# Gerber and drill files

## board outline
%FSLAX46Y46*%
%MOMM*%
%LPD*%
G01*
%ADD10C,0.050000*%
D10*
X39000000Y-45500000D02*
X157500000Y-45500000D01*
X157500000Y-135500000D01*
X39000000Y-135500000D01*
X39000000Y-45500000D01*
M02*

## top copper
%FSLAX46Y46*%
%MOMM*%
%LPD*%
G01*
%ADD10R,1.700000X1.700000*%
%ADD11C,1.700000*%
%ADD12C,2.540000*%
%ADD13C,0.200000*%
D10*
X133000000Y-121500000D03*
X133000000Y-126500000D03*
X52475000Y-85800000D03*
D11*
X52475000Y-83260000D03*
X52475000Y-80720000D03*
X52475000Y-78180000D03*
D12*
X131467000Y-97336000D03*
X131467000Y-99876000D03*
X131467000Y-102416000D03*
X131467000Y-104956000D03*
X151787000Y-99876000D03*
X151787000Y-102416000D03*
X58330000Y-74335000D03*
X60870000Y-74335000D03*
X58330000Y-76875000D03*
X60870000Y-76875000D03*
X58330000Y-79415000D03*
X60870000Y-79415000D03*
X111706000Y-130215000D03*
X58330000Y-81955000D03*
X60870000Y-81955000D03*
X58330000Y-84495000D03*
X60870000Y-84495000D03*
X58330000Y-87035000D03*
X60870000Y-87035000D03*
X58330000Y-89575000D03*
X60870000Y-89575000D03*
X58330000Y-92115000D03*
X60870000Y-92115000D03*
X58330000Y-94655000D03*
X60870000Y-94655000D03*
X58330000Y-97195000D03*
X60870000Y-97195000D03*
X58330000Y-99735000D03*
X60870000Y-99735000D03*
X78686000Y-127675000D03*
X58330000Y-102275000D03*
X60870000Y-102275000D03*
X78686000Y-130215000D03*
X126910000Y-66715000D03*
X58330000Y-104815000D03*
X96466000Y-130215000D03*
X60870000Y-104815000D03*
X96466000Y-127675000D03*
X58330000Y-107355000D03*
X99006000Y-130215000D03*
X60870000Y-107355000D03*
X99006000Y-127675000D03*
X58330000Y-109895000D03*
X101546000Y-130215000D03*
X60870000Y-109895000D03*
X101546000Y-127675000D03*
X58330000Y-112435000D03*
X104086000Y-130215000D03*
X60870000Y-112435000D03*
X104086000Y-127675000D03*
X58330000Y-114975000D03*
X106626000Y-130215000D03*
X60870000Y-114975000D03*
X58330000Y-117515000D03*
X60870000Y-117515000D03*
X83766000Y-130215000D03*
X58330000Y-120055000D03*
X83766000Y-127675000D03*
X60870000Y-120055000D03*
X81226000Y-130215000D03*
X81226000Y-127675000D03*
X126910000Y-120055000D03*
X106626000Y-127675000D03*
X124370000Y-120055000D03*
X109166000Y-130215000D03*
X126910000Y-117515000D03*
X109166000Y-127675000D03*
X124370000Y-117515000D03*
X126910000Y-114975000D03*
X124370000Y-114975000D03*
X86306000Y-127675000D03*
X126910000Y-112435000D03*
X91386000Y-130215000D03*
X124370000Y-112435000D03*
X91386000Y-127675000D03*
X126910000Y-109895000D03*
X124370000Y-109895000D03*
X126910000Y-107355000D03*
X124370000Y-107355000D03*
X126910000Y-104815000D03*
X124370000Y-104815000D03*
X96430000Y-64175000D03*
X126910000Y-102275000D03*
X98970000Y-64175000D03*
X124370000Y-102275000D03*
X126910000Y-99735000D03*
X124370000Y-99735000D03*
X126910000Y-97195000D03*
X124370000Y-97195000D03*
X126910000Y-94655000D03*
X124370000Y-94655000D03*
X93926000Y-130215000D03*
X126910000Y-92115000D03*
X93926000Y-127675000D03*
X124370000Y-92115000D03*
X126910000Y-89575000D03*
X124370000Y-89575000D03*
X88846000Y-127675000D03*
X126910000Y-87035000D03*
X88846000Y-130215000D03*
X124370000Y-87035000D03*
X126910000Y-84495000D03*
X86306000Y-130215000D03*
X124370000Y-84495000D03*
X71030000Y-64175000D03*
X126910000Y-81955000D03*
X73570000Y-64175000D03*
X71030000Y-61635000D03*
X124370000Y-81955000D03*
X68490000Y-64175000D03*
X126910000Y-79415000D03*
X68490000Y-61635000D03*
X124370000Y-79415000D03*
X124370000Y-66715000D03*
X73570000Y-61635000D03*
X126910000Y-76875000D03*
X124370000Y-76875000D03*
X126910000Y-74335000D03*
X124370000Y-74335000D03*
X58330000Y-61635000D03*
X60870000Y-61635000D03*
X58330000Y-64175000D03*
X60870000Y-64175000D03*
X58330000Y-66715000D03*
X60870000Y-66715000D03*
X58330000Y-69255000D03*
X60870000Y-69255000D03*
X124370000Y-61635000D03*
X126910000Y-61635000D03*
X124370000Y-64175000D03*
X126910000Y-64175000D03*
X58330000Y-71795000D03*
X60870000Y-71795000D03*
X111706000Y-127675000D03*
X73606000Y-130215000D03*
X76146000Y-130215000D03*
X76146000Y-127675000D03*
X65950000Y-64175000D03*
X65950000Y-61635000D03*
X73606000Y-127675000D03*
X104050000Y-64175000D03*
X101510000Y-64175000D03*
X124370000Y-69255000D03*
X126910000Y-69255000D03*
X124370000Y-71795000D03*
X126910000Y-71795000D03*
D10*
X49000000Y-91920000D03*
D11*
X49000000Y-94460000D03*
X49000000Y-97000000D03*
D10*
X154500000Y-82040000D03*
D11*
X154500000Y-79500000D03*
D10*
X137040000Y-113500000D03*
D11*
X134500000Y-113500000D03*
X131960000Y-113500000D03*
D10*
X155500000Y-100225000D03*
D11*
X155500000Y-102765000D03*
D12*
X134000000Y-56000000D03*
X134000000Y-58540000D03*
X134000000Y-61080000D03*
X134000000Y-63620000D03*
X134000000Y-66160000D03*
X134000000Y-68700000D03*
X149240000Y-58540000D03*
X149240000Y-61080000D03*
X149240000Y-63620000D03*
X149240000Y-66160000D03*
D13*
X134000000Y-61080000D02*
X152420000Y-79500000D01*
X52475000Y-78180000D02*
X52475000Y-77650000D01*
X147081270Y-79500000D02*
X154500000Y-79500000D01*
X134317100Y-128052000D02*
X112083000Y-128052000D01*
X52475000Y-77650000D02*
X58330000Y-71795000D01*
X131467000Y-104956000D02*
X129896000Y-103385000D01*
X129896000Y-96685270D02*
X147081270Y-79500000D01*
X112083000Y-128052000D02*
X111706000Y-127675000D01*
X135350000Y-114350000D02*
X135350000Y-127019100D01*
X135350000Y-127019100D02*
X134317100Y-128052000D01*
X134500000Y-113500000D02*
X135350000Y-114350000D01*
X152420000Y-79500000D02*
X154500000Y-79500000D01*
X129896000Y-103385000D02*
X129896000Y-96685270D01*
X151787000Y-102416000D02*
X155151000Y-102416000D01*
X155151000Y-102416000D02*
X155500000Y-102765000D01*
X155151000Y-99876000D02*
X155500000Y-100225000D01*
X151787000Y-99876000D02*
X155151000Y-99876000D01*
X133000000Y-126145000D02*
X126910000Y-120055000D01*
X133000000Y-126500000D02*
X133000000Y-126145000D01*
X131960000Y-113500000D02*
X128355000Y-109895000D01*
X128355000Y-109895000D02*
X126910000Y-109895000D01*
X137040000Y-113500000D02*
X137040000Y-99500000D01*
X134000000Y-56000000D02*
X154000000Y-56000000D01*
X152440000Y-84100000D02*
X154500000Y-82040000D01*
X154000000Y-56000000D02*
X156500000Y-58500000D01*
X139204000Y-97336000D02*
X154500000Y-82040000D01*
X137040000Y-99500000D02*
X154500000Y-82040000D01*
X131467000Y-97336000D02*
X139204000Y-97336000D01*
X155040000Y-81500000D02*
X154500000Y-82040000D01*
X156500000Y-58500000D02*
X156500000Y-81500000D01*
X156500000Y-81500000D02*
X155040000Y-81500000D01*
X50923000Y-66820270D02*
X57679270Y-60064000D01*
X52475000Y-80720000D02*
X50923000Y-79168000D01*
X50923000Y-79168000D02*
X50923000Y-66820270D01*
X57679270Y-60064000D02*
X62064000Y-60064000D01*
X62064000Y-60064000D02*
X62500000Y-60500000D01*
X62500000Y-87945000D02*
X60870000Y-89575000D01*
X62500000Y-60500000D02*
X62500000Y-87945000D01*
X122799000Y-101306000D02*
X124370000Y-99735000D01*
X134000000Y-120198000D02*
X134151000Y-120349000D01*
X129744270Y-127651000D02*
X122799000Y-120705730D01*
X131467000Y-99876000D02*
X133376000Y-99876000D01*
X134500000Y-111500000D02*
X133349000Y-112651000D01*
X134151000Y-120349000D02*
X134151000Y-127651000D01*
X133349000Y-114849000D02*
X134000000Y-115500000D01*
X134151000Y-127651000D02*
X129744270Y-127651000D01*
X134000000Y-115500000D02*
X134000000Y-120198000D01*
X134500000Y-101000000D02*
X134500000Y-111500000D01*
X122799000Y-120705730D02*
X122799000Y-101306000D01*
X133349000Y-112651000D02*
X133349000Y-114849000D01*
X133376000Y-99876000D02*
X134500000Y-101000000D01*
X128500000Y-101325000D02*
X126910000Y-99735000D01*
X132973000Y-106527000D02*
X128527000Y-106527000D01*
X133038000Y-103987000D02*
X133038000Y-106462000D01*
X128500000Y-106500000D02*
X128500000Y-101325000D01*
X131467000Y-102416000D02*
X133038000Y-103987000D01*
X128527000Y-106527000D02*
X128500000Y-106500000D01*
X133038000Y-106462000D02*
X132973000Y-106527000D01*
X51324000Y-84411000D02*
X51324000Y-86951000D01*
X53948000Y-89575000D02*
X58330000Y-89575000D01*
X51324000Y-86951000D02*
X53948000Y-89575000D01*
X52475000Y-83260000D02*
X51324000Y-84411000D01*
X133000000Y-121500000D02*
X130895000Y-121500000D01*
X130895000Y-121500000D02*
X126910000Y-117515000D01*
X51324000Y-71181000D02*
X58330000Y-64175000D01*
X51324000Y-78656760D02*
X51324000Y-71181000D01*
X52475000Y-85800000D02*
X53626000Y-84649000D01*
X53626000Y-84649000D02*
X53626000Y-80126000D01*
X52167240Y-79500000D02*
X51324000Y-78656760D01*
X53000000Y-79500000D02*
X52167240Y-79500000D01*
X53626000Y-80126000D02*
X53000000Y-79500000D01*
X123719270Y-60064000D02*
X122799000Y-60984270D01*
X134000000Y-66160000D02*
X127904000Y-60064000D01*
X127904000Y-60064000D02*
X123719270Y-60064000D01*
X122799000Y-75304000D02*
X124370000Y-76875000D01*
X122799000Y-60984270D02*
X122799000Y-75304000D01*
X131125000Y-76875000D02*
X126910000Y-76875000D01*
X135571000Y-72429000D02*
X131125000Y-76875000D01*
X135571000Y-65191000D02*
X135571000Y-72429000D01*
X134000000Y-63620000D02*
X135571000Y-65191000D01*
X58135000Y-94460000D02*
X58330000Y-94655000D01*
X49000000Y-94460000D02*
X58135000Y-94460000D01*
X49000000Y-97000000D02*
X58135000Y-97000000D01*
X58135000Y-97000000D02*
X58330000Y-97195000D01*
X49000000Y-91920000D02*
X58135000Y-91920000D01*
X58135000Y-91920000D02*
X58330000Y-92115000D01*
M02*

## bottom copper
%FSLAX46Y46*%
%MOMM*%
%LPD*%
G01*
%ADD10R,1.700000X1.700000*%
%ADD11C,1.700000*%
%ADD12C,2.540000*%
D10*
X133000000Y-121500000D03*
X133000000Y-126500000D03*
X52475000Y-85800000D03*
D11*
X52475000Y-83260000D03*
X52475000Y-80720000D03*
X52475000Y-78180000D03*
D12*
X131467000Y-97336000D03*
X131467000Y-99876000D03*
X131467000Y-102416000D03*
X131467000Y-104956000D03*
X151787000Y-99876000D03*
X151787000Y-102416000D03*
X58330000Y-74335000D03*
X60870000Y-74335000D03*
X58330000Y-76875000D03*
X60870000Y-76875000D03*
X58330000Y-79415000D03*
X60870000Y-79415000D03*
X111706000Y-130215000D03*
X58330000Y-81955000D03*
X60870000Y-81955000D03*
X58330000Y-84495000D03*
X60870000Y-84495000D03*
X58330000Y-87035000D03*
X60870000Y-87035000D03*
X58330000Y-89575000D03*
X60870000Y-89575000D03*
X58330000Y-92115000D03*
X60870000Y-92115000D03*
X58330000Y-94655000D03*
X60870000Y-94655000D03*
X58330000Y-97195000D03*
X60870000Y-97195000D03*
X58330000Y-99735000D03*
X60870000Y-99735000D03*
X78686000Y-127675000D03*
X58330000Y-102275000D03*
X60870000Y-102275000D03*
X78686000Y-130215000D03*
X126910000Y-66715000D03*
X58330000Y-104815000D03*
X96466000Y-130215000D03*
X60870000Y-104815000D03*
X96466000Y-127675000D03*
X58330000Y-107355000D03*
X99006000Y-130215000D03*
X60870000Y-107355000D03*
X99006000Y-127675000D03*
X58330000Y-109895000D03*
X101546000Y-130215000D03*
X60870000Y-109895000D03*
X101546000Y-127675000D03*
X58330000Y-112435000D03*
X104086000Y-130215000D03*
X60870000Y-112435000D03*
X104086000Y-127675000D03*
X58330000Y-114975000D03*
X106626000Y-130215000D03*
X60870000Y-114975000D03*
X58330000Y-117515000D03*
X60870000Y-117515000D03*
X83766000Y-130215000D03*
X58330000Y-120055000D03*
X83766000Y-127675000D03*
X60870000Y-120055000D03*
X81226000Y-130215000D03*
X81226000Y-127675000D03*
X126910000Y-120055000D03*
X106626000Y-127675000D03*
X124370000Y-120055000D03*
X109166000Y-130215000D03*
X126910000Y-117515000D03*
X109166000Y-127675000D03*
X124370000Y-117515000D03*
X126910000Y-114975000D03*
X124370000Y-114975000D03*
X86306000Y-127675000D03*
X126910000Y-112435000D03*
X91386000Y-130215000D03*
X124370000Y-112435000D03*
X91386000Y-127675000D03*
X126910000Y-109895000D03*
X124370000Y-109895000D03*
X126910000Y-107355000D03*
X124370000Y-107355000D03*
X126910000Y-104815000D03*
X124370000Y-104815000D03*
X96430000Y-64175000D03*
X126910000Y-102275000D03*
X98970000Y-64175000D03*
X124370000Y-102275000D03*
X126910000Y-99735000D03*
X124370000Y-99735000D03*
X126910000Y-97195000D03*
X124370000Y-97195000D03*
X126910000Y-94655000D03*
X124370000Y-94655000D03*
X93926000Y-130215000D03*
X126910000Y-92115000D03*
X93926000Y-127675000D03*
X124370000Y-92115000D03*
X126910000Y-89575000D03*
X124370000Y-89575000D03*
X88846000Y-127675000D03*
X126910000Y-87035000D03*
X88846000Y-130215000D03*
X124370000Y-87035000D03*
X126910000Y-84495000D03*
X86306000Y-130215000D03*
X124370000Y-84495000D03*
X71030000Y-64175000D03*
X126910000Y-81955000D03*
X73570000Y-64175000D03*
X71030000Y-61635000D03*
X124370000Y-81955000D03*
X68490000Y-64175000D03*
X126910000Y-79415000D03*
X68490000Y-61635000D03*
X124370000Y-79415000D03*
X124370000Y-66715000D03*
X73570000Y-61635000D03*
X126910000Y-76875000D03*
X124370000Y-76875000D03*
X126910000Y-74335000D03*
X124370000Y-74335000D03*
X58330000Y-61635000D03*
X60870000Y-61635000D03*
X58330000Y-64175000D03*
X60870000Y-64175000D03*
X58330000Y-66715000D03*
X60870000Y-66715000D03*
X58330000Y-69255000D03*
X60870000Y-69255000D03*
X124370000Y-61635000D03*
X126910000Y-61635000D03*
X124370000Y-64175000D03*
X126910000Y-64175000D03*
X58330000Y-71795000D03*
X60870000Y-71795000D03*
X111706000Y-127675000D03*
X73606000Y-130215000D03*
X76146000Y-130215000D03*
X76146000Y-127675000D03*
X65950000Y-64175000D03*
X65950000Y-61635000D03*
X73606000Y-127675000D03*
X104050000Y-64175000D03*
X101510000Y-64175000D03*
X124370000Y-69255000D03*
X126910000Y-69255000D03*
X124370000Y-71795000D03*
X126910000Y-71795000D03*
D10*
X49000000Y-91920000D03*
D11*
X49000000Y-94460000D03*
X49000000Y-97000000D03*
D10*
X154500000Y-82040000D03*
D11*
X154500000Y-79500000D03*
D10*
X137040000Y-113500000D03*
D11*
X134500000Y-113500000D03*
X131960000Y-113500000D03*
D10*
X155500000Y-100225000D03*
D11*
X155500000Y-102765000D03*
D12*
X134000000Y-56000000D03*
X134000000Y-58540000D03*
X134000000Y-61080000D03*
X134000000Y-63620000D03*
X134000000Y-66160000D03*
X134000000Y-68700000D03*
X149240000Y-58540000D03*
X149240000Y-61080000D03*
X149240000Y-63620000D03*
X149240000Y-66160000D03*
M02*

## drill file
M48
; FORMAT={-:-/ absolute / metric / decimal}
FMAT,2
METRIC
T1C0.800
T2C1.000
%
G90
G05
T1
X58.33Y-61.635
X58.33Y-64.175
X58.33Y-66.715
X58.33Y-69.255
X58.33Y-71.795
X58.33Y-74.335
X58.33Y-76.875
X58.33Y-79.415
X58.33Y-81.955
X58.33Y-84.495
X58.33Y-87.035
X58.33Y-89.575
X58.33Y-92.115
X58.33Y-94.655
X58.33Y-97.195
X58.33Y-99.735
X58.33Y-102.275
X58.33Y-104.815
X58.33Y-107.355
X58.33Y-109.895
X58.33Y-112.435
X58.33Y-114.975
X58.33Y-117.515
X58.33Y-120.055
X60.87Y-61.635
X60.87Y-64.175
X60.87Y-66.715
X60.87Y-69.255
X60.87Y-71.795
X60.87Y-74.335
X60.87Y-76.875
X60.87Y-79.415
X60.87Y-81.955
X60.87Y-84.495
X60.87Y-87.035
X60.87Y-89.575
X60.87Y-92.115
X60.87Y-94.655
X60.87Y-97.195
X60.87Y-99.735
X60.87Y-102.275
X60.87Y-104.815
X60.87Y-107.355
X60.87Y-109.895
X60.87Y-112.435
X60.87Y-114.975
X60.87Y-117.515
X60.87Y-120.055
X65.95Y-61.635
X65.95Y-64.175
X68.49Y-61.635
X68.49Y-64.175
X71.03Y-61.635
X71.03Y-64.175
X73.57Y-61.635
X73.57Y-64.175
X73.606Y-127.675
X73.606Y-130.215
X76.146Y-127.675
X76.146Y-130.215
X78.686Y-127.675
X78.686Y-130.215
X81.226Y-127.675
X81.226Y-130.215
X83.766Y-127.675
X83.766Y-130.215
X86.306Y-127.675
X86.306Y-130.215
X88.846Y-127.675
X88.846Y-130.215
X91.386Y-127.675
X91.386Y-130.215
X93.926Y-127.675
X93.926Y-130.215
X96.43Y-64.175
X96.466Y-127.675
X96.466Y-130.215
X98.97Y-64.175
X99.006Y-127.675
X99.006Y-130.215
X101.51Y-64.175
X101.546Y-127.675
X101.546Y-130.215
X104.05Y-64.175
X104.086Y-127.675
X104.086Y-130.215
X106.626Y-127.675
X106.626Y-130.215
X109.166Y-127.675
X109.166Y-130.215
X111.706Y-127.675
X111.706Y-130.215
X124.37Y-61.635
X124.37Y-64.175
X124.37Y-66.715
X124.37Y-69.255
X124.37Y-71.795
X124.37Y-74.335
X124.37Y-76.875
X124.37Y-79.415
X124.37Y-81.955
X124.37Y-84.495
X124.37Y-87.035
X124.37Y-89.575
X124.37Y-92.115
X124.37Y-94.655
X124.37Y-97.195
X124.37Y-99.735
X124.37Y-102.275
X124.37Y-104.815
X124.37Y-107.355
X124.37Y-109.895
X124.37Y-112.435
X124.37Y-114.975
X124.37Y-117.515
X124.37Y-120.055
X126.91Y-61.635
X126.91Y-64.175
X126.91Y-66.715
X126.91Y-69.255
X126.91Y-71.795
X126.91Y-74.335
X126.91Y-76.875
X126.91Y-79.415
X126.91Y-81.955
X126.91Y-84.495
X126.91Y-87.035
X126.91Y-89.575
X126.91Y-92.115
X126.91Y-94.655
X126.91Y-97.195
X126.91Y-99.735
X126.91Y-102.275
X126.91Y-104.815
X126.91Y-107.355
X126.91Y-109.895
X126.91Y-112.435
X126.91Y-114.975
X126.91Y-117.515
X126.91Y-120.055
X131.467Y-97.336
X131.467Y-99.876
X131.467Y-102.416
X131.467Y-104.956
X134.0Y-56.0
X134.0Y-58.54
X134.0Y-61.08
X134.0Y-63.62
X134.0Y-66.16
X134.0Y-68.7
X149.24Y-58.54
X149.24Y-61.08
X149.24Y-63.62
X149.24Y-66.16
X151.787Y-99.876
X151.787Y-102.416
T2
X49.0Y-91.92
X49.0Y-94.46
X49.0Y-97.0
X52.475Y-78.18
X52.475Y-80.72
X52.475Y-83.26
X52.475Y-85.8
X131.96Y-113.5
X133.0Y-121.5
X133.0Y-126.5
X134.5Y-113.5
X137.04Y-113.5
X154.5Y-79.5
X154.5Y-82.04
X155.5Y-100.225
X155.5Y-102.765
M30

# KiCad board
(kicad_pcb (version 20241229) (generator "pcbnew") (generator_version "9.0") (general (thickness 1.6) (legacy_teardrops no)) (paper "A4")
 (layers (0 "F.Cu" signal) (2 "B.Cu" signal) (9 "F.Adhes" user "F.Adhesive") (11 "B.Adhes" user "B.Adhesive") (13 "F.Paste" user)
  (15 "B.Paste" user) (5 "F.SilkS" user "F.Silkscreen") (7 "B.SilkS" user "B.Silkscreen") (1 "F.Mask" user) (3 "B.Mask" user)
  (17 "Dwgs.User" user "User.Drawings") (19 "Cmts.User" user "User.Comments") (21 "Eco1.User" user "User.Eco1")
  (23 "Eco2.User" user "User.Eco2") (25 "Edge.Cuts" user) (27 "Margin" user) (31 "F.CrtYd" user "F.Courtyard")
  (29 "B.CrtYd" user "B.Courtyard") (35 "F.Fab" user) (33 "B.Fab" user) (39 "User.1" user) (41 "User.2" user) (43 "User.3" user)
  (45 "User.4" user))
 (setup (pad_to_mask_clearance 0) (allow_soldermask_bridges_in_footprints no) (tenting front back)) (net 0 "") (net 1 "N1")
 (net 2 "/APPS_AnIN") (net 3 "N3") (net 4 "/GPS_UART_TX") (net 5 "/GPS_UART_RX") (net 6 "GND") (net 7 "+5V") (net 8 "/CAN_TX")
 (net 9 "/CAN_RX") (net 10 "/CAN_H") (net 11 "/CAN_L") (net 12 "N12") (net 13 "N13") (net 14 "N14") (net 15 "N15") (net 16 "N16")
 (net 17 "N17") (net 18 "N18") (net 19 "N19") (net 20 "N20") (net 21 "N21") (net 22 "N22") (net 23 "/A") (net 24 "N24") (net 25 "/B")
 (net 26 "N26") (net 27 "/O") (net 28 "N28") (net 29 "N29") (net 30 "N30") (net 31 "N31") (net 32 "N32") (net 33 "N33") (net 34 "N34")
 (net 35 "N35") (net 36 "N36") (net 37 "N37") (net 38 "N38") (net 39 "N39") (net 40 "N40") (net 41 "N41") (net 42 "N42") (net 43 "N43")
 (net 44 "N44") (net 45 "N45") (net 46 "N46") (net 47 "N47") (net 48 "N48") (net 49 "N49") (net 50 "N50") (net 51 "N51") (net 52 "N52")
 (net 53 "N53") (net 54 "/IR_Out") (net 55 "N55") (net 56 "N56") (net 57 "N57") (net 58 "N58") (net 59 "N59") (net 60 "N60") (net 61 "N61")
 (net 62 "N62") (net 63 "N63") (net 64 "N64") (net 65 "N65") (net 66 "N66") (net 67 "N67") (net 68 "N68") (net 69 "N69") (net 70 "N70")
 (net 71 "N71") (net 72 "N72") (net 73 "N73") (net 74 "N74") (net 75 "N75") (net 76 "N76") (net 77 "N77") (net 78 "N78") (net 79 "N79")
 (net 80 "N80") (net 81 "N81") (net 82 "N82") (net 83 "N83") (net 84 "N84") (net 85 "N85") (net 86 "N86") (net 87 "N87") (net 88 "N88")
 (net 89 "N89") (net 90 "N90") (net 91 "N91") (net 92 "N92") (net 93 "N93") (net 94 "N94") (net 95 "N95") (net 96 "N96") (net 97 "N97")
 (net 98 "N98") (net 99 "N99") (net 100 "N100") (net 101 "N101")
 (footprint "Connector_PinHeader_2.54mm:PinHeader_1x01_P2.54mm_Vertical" (layer "F.Cu") (at 133 121.5)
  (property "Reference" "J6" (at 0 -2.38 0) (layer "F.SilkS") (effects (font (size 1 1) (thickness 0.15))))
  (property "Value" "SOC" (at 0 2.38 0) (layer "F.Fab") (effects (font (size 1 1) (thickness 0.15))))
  (pad "1" thru_hole rect (at 0 0) (size 1.7 1.7) (drill 1) (layers "*.Cu" "*.Mask") (remove_unused_layers no) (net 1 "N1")))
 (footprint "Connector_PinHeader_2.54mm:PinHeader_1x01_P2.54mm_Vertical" (layer "F.Cu") (at 133 126.5)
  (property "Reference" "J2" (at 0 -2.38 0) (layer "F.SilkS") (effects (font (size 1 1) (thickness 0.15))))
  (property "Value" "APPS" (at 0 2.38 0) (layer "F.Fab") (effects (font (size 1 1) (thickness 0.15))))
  (pad "1" thru_hole rect (at 0 0) (size 1.7 1.7) (drill 1) (layers "*.Cu" "*.Mask") (remove_unused_layers no) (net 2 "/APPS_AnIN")))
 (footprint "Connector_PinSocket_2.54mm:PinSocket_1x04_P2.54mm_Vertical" (layer "F.Cu") (at 52.475 85.8 180)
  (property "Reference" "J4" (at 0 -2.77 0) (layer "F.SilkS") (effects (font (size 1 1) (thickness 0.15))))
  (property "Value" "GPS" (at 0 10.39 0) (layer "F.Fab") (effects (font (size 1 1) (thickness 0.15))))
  (pad "1" thru_hole rect (at 0 0 180) (size 1.7 1.7) (drill 1) (layers "*.Cu" "*.Mask") (remove_unused_layers no) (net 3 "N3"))
  (pad "2" thru_hole circle (at 0 2.54 180) (size 1.7 1.7) (drill 1) (layers "*.Cu" "*.Mask") (remove_unused_layers no)
   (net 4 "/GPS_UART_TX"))
  (pad "3" thru_hole circle (at 0 5.08 180) (size 1.7 1.7) (drill 1) (layers "*.Cu" "*.Mask") (remove_unused_layers no)
   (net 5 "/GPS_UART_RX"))
  (pad "4" thru_hole circle (at 0 7.62 180) (size 1.7 1.7) (drill 1) (layers "*.Cu" "*.Mask") (remove_unused_layers no) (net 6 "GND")))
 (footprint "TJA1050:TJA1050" (layer "F.Cu") (at 141.627 107.242)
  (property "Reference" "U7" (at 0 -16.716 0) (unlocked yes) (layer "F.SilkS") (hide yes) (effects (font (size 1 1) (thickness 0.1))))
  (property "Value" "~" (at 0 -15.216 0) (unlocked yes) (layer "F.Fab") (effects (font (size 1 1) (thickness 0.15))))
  (pad "1" thru_hole circle (at -10.16 -9.906) (size 2.54 2.54) (drill 0.8) (layers "*.Cu" "*.Mask") (remove_unused_layers no) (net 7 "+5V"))
  (pad "2" thru_hole circle (at -10.16 -7.366) (size 2.54 2.54) (drill 0.8) (layers "*.Cu" "*.Mask") (remove_unused_layers no)
   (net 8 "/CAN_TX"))
  (pad "3" thru_hole circle (at -10.16 -4.826) (size 2.54 2.54) (drill 0.8) (layers "*.Cu" "*.Mask") (remove_unused_layers no)
   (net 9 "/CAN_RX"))
  (pad "4" thru_hole circle (at -10.16 -2.286) (size 2.54 2.54) (drill 0.8) (layers "*.Cu" "*.Mask") (remove_unused_layers no) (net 6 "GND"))
  (pad "5" thru_hole circle (at 10.16 -7.366) (size 2.54 2.54) (drill 0.8) (layers "*.Cu" "*.Mask") (remove_unused_layers no)
   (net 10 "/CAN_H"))
  (pad "6" thru_hole circle (at 10.16 -4.826) (size 2.54 2.54) (drill 0.8) (layers "*.Cu" "*.Mask") (remove_unused_layers no)
   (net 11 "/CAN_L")))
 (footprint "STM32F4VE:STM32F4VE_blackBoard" (layer "F.Cu") (at 92.62 89.575)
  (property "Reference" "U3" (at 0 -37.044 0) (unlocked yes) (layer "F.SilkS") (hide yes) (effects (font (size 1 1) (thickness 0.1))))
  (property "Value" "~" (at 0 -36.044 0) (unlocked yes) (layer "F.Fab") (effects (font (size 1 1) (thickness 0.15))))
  (pad "1" thru_hole circle (at -34.29 -15.24) (size 2.54 2.54) (drill 0.8) (layers "*.Cu" "*.Mask") (remove_unused_layers no)
   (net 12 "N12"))
  (pad "2" thru_hole circle (at -31.75 -15.24) (size 2.54 2.54) (drill 0.8) (layers "*.Cu" "*.Mask") (remove_unused_layers no)
   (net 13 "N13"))
  (pad "3" thru_hole circle (at -34.29 -12.7) (size 2.54 2.54) (drill 0.8) (layers "*.Cu" "*.Mask") (remove_unused_layers no) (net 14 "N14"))
  (pad "4" thru_hole circle (at -31.75 -12.7) (size 2.54 2.54) (drill 0.8) (layers "*.Cu" "*.Mask") (remove_unused_layers no) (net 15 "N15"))
  (pad "5" thru_hole circle (at -34.29 -10.16) (size 2.54 2.54) (drill 0.8) (layers "*.Cu" "*.Mask") (remove_unused_layers no)
   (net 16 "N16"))
  (pad "7" thru_hole circle (at -31.75 -10.16) (size 2.54 2.54) (drill 0.8) (layers "*.Cu" "*.Mask") (remove_unused_layers no)
   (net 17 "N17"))
  (pad "14" thru_hole circle (at 19.086 40.64) (size 2.54 2.54) (drill 0.8) (layers "*.Cu" "*.Mask") (remove_unused_layers no)
   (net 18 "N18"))
  (pad "15" thru_hole circle (at -34.29 -7.62) (size 2.54 2.54) (drill 0.8) (layers "*.Cu" "*.Mask") (remove_unused_layers no)
   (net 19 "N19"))
  (pad "16" thru_hole circle (at -31.75 -7.62) (size 2.54 2.54) (drill 0.8) (layers "*.Cu" "*.Mask") (remove_unused_layers no)
   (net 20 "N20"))
  (pad "17" thru_hole circle (at -34.29 -5.08) (size 2.54 2.54) (drill 0.8) (layers "*.Cu" "*.Mask") (remove_unused_layers no)
   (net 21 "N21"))
  (pad "18" thru_hole circle (at -31.75 -5.08) (size 2.54 2.54) (drill 0.8) (layers "*.Cu" "*.Mask") (remove_unused_layers no)
   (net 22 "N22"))
  (pad "20" thru_hole circle (at -34.29 -2.54) (size 2.54 2.54) (drill 0.8) (layers "*.Cu" "*.Mask") (remove_unused_layers no))
  (pad "21" thru_hole circle (at -31.75 -2.54) (size 2.54 2.54) (drill 0.8) (layers "*.Cu" "*.Mask") (remove_unused_layers no))
  (pad "23" thru_hole circle (at -34.29 0) (size 2.54 2.54) (drill 0.8) (layers "*.Cu" "*.Mask") (remove_unused_layers no)
   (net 4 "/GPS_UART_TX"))
  (pad "24" thru_hole circle (at -31.75 0) (size 2.54 2.54) (drill 0.8) (layers "*.Cu" "*.Mask") (remove_unused_layers no)
   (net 5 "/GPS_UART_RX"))
  (pad "25" thru_hole circle (at -34.29 2.54) (size 2.54 2.54) (drill 0.8) (layers "*.Cu" "*.Mask") (remove_unused_layers no) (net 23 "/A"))
  (pad "26" thru_hole circle (at -31.75 2.54) (size 2.54 2.54) (drill 0.8) (layers "*.Cu" "*.Mask") (remove_unused_layers no) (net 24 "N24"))
  (pad "29" thru_hole circle (at -34.29 5.08) (size 2.54 2.54) (drill 0.8) (layers "*.Cu" "*.Mask") (remove_unused_layers no) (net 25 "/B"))
  (pad "30" thru_hole circle (at -31.75 5.08) (size 2.54 2.54) (drill 0.8) (layers "*.Cu" "*.Mask") (remove_unused_layers no) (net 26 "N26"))
  (pad "31" thru_hole circle (at -34.29 7.62) (size 2.54 2.54) (drill 0.8) (layers "*.Cu" "*.Mask") (remove_unused_layers no) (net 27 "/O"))
  (pad "32" thru_hole circle (at -31.75 7.62) (size 2.54 2.54) (drill 0.8) (layers "*.Cu" "*.Mask") (remove_unused_layers no) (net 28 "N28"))
  (pad "33" thru_hole circle (at -34.29 10.16) (size 2.54 2.54) (drill 0.8) (layers "*.Cu" "*.Mask") (remove_unused_layers no)
   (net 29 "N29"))
  (pad "34" thru_hole circle (at -31.75 10.16) (size 2.54 2.54) (drill 0.8) (layers "*.Cu" "*.Mask") (remove_unused_layers no)
   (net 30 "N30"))
  (pad "34" thru_hole circle (at -13.934 38.1) (size 2.54 2.54) (drill 0.8) (layers "*.Cu" "*.Mask") (remove_unused_layers no)
   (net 30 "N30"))
  (pad "35" thru_hole circle (at -34.29 12.7) (size 2.54 2.54) (drill 0.8) (layers "*.Cu" "*.Mask") (remove_unused_layers no) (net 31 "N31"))
  (pad "36" thru_hole circle (at -31.75 12.7) (size 2.54 2.54) (drill 0.8) (layers "*.Cu" "*.Mask") (remove_unused_layers no) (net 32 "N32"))
  (pad "36" thru_hole circle (at -13.934 40.64) (size 2.54 2.54) (drill 0.8) (layers "*.Cu" "*.Mask") (remove_unused_layers no)
   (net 32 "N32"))
  (pad "37" thru_hole circle (at 34.29 -22.86) (size 2.54 2.54) (drill 0.8) (layers "*.Cu" "*.Mask") (remove_unused_layers no)
   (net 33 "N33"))
  (pad "38" thru_hole circle (at -34.29 15.24) (size 2.54 2.54) (drill 0.8) (layers "*.Cu" "*.Mask") (remove_unused_layers no)
   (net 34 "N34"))
  (pad "38" thru_hole circle (at 3.846 40.64) (size 2.54 2.54) (drill 0.8) (layers "*.Cu" "*.Mask") (remove_unused_layers no) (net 34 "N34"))
  (pad "39" thru_hole circle (at -31.75 15.24) (size 2.54 2.54) (drill 0.8) (layers "*.Cu" "*.Mask") (remove_unused_layers no)
   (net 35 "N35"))
  (pad "39" thru_hole circle (at 3.846 38.1) (size 2.54 2.54) (drill 0.8) (layers "*.Cu" "*.Mask") (remove_unused_layers no) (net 35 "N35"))
  (pad "40" thru_hole circle (at -34.29 17.78) (size 2.54 2.54) (drill 0.8) (layers "*.Cu" "*.Mask") (remove_unused_layers no)
   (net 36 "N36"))
  (pad "40" thru_hole circle (at 6.386 40.64) (size 2.54 2.54) (drill 0.8) (layers "*.Cu" "*.Mask") (remove_unused_layers no) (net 36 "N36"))
  (pad "41" thru_hole circle (at -31.75 17.78) (size 2.54 2.54) (drill 0.8) (layers "*.Cu" "*.Mask") (remove_unused_layers no)
   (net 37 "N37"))
  (pad "41" thru_hole circle (at 6.386 38.1) (size 2.54 2.54) (drill 0.8) (layers "*.Cu" "*.Mask") (remove_unused_layers no) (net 37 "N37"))
  (pad "42" thru_hole circle (at -34.29 20.32) (size 2.54 2.54) (drill 0.8) (layers "*.Cu" "*.Mask") (remove_unused_layers no)
   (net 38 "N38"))
  (pad "42" thru_hole circle (at 8.926 40.64) (size 2.54 2.54) (drill 0.8) (layers "*.Cu" "*.Mask") (remove_unused_layers no) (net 38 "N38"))
  (pad "43" thru_hole circle (at -31.75 20.32) (size 2.54 2.54) (drill 0.8) (layers "*.Cu" "*.Mask") (remove_unused_layers no)
   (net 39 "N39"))
  (pad "43" thru_hole circle (at 8.926 38.1) (size 2.54 2.54) (drill 0.8) (layers "*.Cu" "*.Mask") (remove_unused_layers no) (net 39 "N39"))
  (pad "44" thru_hole circle (at -34.29 22.86) (size 2.54 2.54) (drill 0.8) (layers "*.Cu" "*.Mask") (remove_unused_layers no)
   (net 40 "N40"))
  (pad "44" thru_hole circle (at 11.466 40.64) (size 2.54 2.54) (drill 0.8) (layers "*.Cu" "*.Mask") (remove_unused_layers no)
   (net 40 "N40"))
  (pad "45" thru_hole circle (at -31.75 22.86) (size 2.54 2.54) (drill 0.8) (layers "*.Cu" "*.Mask") (remove_unused_layers no)
   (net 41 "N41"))
  (pad "45" thru_hole circle (at 11.466 38.1) (size 2.54 2.54) (drill 0.8) (layers "*.Cu" "*.Mask") (remove_unused_layers no) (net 41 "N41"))
  (pad "46" thru_hole circle (at -34.29 25.4) (size 2.54 2.54) (drill 0.8) (layers "*.Cu" "*.Mask") (remove_unused_layers no) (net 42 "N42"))
  (pad "46" thru_hole circle (at 14.006 40.64) (size 2.54 2.54) (drill 0.8) (layers "*.Cu" "*.Mask") (remove_unused_layers no)
   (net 42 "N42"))
  (pad "47" thru_hole circle (at -31.75 25.4) (size 2.54 2.54) (drill 0.8) (layers "*.Cu" "*.Mask") (remove_unused_layers no) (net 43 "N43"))
  (pad "48" thru_hole circle (at -34.29 27.94) (size 2.54 2.54) (drill 0.8) (layers "*.Cu" "*.Mask") (remove_unused_layers no)
   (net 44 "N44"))
  (pad "51" thru_hole circle (at -31.75 27.94) (size 2.54 2.54) (drill 0.8) (layers "*.Cu" "*.Mask") (remove_unused_layers no)
   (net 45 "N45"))
  (pad "51" thru_hole circle (at -8.854 40.64) (size 2.54 2.54) (drill 0.8) (layers "*.Cu" "*.Mask") (remove_unused_layers no)
   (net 45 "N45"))
  (pad "52" thru_hole circle (at -34.29 30.48) (size 2.54 2.54) (drill 0.8) (layers "*.Cu" "*.Mask") (remove_unused_layers no)
   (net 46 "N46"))
  (pad "52" thru_hole circle (at -8.854 38.1) (size 2.54 2.54) (drill 0.8) (layers "*.Cu" "*.Mask") (remove_unused_layers no) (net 46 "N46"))
  (pad "53" thru_hole circle (at -31.75 30.48) (size 2.54 2.54) (drill 0.8) (layers "*.Cu" "*.Mask") (remove_unused_layers no)
   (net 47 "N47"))
  (pad "53" thru_hole circle (at -11.394 40.64) (size 2.54 2.54) (drill 0.8) (layers "*.Cu" "*.Mask") (remove_unused_layers no)
   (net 47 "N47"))
  (pad "54" thru_hole circle (at -11.394 38.1) (size 2.54 2.54) (drill 0.8) (layers "*.Cu" "*.Mask") (remove_unused_layers no)
   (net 2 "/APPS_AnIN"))
  (pad "54" thru_hole circle (at 34.29 30.48) (size 2.54 2.54) (drill 0.8) (layers "*.Cu" "*.Mask") (remove_unused_layers no)
   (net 2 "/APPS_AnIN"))
  (pad "55" thru_hole circle (at 14.006 38.1) (size 2.54 2.54) (drill 0.8) (layers "*.Cu" "*.Mask") (remove_unused_layers no) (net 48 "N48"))
  (pad "55" thru_hole circle (at 31.75 30.48) (size 2.54 2.54) (drill 0.8) (layers "*.Cu" "*.Mask") (remove_unused_layers no) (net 48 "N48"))
  (pad "56" thru_hole circle (at 16.546 40.64) (size 2.54 2.54) (drill 0.8) (layers "*.Cu" "*.Mask") (remove_unused_layers no) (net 1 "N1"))
  (pad "56" thru_hole circle (at 34.29 27.94) (size 2.54 2.54) (drill 0.8) (layers "*.Cu" "*.Mask") (remove_unused_layers no) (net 1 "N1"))
  (pad "57" thru_hole circle (at 16.546 38.1) (size 2.54 2.54) (drill 0.8) (layers "*.Cu" "*.Mask") (remove_unused_layers no) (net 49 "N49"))
  (pad "57" thru_hole circle (at 31.75 27.94) (size 2.54 2.54) (drill 0.8) (layers "*.Cu" "*.Mask") (remove_unused_layers no) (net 49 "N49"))
  (pad "58" thru_hole circle (at 34.29 25.4) (size 2.54 2.54) (drill 0.8) (layers "*.Cu" "*.Mask") (remove_unused_layers no) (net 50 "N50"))
  (pad "59" thru_hole circle (at 31.75 25.4) (size 2.54 2.54) (drill 0.8) (layers "*.Cu" "*.Mask") (remove_unused_layers no) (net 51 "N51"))
  (pad "60" thru_hole circle (at -6.314 38.1) (size 2.54 2.54) (drill 0.8) (layers "*.Cu" "*.Mask") (remove_unused_layers no) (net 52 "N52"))
  (pad "60" thru_hole circle (at 34.29 22.86) (size 2.54 2.54) (drill 0.8) (layers "*.Cu" "*.Mask") (remove_unused_layers no) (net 52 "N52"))
  (pad "61" thru_hole circle (at -1.234 40.64) (size 2.54 2.54) (drill 0.8) (layers "*.Cu" "*.Mask") (remove_unused_layers no)
   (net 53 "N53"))
  (pad "61" thru_hole circle (at 31.75 22.86) (size 2.54 2.54) (drill 0.8) (layers "*.Cu" "*.Mask") (remove_unused_layers no) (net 53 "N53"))
  (pad "62" thru_hole circle (at -1.234 38.1) (size 2.54 2.54) (drill 0.8) (layers "*.Cu" "*.Mask") (remove_unused_layers no)
   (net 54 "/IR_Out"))
  (pad "62" thru_hole circle (at 34.29 20.32) (size 2.54 2.54) (drill 0.8) (layers "*.Cu" "*.Mask") (remove_unused_layers no)
   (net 54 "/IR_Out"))
  (pad "63" thru_hole circle (at 31.75 20.32) (size 2.54 2.54) (drill 0.8) (layers "*.Cu" "*.Mask") (remove_unused_layers no) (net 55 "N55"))
  (pad "64" thru_hole circle (at 34.29 17.78) (size 2.54 2.54) (drill 0.8) (layers "*.Cu" "*.Mask") (remove_unused_layers no) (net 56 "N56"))
  (pad "65" thru_hole circle (at 31.75 17.78) (size 2.54 2.54) (drill 0.8) (layers "*.Cu" "*.Mask") (remove_unused_layers no) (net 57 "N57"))
  (pad "66" thru_hole circle (at 34.29 15.24) (size 2.54 2.54) (drill 0.8) (layers "*.Cu" "*.Mask") (remove_unused_layers no) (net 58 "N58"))
  (pad "67" thru_hole circle (at 31.75 15.24) (size 2.54 2.54) (drill 0.8) (layers "*.Cu" "*.Mask") (remove_unused_layers no) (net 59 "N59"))
  (pad "68" thru_hole circle (at 3.81 -25.4) (size 2.54 2.54) (drill 0.8) (layers "*.Cu" "*.Mask") (remove_unused_layers no) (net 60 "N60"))
  (pad "68" thru_hole circle (at 34.29 12.7) (size 2.54 2.54) (drill 0.8) (layers "*.Cu" "*.Mask") (remove_unused_layers no) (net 60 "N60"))
  (pad "69" thru_hole circle (at 6.35 -25.4) (size 2.54 2.54) (drill 0.8) (layers "*.Cu" "*.Mask") (remove_unused_layers no) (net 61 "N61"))
  (pad "69" thru_hole circle (at 31.75 12.7) (size 2.54 2.54) (drill 0.8) (layers "*.Cu" "*.Mask") (remove_unused_layers no) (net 61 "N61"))
  (pad "70" thru_hole circle (at 34.29 10.16) (size 2.54 2.54) (drill 0.8) (layers "*.Cu" "*.Mask") (remove_unused_layers no)
   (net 9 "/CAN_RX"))
  (pad "71" thru_hole circle (at 31.75 10.16) (size 2.54 2.54) (drill 0.8) (layers "*.Cu" "*.Mask") (remove_unused_layers no)
   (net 8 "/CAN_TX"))
  (pad "77" thru_hole circle (at 34.29 7.62) (size 2.54 2.54) (drill 0.8) (layers "*.Cu" "*.Mask") (remove_unused_layers no) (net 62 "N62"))
  (pad "78" thru_hole circle (at 31.75 7.62) (size 2.54 2.54) (drill 0.8) (layers "*.Cu" "*.Mask") (remove_unused_layers no) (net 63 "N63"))
  (pad "79" thru_hole circle (at 34.29 5.08) (size 2.54 2.54) (drill 0.8) (layers "*.Cu" "*.Mask") (remove_unused_layers no) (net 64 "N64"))
  (pad "80" thru_hole circle (at 31.75 5.08) (size 2.54 2.54) (drill 0.8) (layers "*.Cu" "*.Mask") (remove_unused_layers no) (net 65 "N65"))
  (pad "81" thru_hole circle (at 1.306 40.64) (size 2.54 2.54) (drill 0.8) (layers "*.Cu" "*.Mask") (remove_unused_layers no) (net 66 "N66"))
  (pad "81" thru_hole circle (at 34.29 2.54) (size 2.54 2.54) (drill 0.8) (layers "*.Cu" "*.Mask") (remove_unused_layers no) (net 66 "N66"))
  (pad "82" thru_hole circle (at 1.306 38.1) (size 2.54 2.54) (drill 0.8) (layers "*.Cu" "*.Mask") (remove_unused_layers no) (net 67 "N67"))
  (pad "82" thru_hole circle (at 31.75 2.54) (size 2.54 2.54) (drill 0.8) (layers "*.Cu" "*.Mask") (remove_unused_layers no) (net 67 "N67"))
  (pad "83" thru_hole circle (at 34.29 0) (size 2.54 2.54) (drill 0.8) (layers "*.Cu" "*.Mask") (remove_unused_layers no) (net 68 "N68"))
  (pad "84" thru_hole circle (at 31.75 0) (size 2.54 2.54) (drill 0.8) (layers "*.Cu" "*.Mask") (remove_unused_layers no) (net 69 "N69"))
  (pad "85" thru_hole circle (at -3.774 38.1) (size 2.54 2.54) (drill 0.8) (layers "*.Cu" "*.Mask") (remove_unused_layers no) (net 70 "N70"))
  (pad "85" thru_hole circle (at 34.29 -2.54) (size 2.54 2.54) (drill 0.8) (layers "*.Cu" "*.Mask") (remove_unused_layers no) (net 70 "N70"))
  (pad "86" thru_hole circle (at -3.774 40.64) (size 2.54 2.54) (drill 0.8) (layers "*.Cu" "*.Mask") (remove_unused_layers no)
   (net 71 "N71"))
  (pad "86" thru_hole circle (at 31.75 -2.54) (size 2.54 2.54) (drill 0.8) (layers "*.Cu" "*.Mask") (remove_unused_layers no) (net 71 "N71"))
  (pad "87" thru_hole circle (at 34.29 -5.08) (size 2.54 2.54) (drill 0.8) (layers "*.Cu" "*.Mask") (remove_unused_layers no) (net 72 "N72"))
  (pad "88" thru_hole circle (at -6.314 40.64) (size 2.54 2.54) (drill 0.8) (layers "*.Cu" "*.Mask") (remove_unused_layers no)
   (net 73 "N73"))
  (pad "88" thru_hole circle (at 31.75 -5.08) (size 2.54 2.54) (drill 0.8) (layers "*.Cu" "*.Mask") (remove_unused_layers no) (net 73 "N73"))
  (pad "89" thru_hole circle (at -21.59 -25.4) (size 2.54 2.54) (drill 0.8) (layers "*.Cu" "*.Mask") (remove_unused_layers no)
   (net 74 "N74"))
  (pad "89" thru_hole circle (at 34.29 -7.62) (size 2.54 2.54) (drill 0.8) (layers "*.Cu" "*.Mask") (remove_unused_layers no) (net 74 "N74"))
  (pad "90" thru_hole circle (at -19.05 -25.4) (size 2.54 2.54) (drill 0.8) (layers "*.Cu" "*.Mask") (remove_unused_layers no)
   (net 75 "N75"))
  (pad "91" thru_hole circle (at -21.59 -27.94) (size 2.54 2.54) (drill 0.8) (layers "*.Cu" "*.Mask") (remove_unused_layers no)
   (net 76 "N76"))
  (pad "91" thru_hole circle (at 31.75 -7.62) (size 2.54 2.54) (drill 0.8) (layers "*.Cu" "*.Mask") (remove_unused_layers no) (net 76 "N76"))
  (pad "92" thru_hole circle (at -24.13 -25.4) (size 2.54 2.54) (drill 0.8) (layers "*.Cu" "*.Mask") (remove_unused_layers no)
   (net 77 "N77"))
  (pad "92" thru_hole circle (at 34.29 -10.16) (size 2.54 2.54) (drill 0.8) (layers "*.Cu" "*.Mask") (remove_unused_layers no)
   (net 77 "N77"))
  (pad "93" thru_hole circle (at -24.13 -27.94) (size 2.54 2.54) (drill 0.8) (layers "*.Cu" "*.Mask") (remove_unused_layers no)
   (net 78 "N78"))
  (pad "93" thru_hole circle (at 31.75 -10.16) (size 2.54 2.54) (drill 0.8) (layers "*.Cu" "*.Mask") (remove_unused_layers no)
   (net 78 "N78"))
  (pad "94" thru_hole circle (at 31.75 -22.86) (size 2.54 2.54) (drill 0.8) (layers "*.Cu" "*.Mask") (remove_unused_layers no)
   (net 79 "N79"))
  (pad "95" thru_hole circle (at -19.05 -27.94) (size 2.54 2.54) (drill 0.8) (layers "*.Cu" "*.Mask") (remove_unused_layers no)
   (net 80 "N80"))
  (pad "95" thru_hole circle (at 34.29 -12.7) (size 2.54 2.54) (drill 0.8) (layers "*.Cu" "*.Mask") (remove_unused_layers no) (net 80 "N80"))
  (pad "96" thru_hole circle (at 31.75 -12.7) (size 2.54 2.54) (drill 0.8) (layers "*.Cu" "*.Mask") (remove_unused_layers no) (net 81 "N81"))
  (pad "97" thru_hole circle (at 34.29 -15.24) (size 2.54 2.54) (drill 0.8) (layers "*.Cu" "*.Mask") (remove_unused_layers no)
   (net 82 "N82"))
  (pad "98" thru_hole circle (at 31.75 -15.24) (size 2.54 2.54) (drill 0.8) (layers "*.Cu" "*.Mask") (remove_unused_layers no)
   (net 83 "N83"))
  (pad "101" thru_hole circle (at -34.29 -27.94) (size 2.54 2.54) (drill 0.8) (layers "*.Cu" "*.Mask") (remove_unused_layers no)
   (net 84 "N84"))
  (pad "102" thru_hole circle (at -31.75 -27.94) (size 2.54 2.54) (drill 0.8) (layers "*.Cu" "*.Mask") (remove_unused_layers no)
   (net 7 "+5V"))
  (pad "103" thru_hole circle (at -34.29 -25.4) (size 2.54 2.54) (drill 0.8) (layers "*.Cu" "*.Mask") (remove_unused_layers no) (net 3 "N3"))
  (pad "104" thru_hole circle (at -31.75 -25.4) (size 2.54 2.54) (drill 0.8) (layers "*.Cu" "*.Mask") (remove_unused_layers no)
   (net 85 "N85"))
  (pad "111" thru_hole circle (at -34.29 -22.86) (size 2.54 2.54) (drill 0.8) (layers "*.Cu" "*.Mask") (remove_unused_layers no)
   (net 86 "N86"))
  (pad "112" thru_hole circle (at -31.75 -22.86) (size 2.54 2.54) (drill 0.8) (layers "*.Cu" "*.Mask") (remove_unused_layers no)
   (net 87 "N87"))
  (pad "113" thru_hole circle (at -34.29 -20.32) (size 2.54 2.54) (drill 0.8) (layers "*.Cu" "*.Mask") (remove_unused_layers no)
   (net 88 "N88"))
  (pad "114" thru_hole circle (at -31.75 -20.32) (size 2.54 2.54) (drill 0.8) (layers "*.Cu" "*.Mask") (remove_unused_layers no)
   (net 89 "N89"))
  (pad "115" thru_hole circle (at 31.75 -27.94) (size 2.54 2.54) (drill 0.8) (layers "*.Cu" "*.Mask") (remove_unused_layers no)
   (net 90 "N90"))
  (pad "116" thru_hole circle (at 34.29 -27.94) (size 2.54 2.54) (drill 0.8) (layers "*.Cu" "*.Mask") (remove_unused_layers no)
   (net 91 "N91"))
  (pad "117" thru_hole circle (at 31.75 -25.4) (size 2.54 2.54) (drill 0.8) (layers "*.Cu" "*.Mask") (remove_unused_layers no)
   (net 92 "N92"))
  (pad "118" thru_hole circle (at 34.29 -25.4) (size 2.54 2.54) (drill 0.8) (layers "*.Cu" "*.Mask") (remove_unused_layers no)
   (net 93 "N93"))
  (pad "121" thru_hole circle (at -34.29 -17.78) (size 2.54 2.54) (drill 0.8) (layers "*.Cu" "*.Mask") (remove_unused_layers no)
   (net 6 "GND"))
  (pad "122" thru_hole circle (at -31.75 -17.78) (size 2.54 2.54) (drill 0.8) (layers "*.Cu" "*.Mask") (remove_unused_layers no)
   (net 6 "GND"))
  (pad "201" thru_hole circle (at 19.086 38.1) (size 2.54 2.54) (drill 0.8) (layers "*.Cu" "*.Mask") (remove_unused_layers no) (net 6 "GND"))
  (pad "202" thru_hole circle (at -19.014 40.64) (size 2.54 2.54) (drill 0.8) (layers "*.Cu" "*.Mask") (remove_unused_layers no)
   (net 6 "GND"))
  (pad "203" thru_hole circle (at -16.474 40.64) (size 2.54 2.54) (drill 0.8) (layers "*.Cu" "*.Mask") (remove_unused_layers no)
   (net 6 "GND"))
  (pad "229" thru_hole circle (at -16.474 38.1) (size 2.54 2.54) (drill 0.8) (layers "*.Cu" "*.Mask") (remove_unused_layers no)
   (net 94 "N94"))
  (pad "241" thru_hole circle (at -26.67 -25.4) (size 2.54 2.54) (drill 0.8) (layers "*.Cu" "*.Mask") (remove_unused_layers no)
   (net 6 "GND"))
  (pad "242" thru_hole circle (at -26.67 -27.94) (size 2.54 2.54) (drill 0.8) (layers "*.Cu" "*.Mask") (remove_unused_layers no)
   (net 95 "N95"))
  (pad "243" thru_hole circle (at -19.014 38.1) (size 2.54 2.54) (drill 0.8) (layers "*.Cu" "*.Mask") (remove_unused_layers no)
   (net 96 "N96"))
  (pad "251" thru_hole circle (at 11.43 -25.4) (size 2.54 2.54) (drill 0.8) (layers "*.Cu" "*.Mask") (remove_unused_layers no)
   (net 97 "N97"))
  (pad "252" thru_hole circle (at 8.89 -25.4) (size 2.54 2.54) (drill 0.8) (layers "*.Cu" "*.Mask") (remove_unused_layers no) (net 6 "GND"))
  (pad "260" thru_hole circle (at 31.75 -20.32) (size 2.54 2.54) (drill 0.8) (layers "*.Cu" "*.Mask") (remove_unused_layers no)
   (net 6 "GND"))
  (pad "261" thru_hole circle (at 34.29 -20.32) (size 2.54 2.54) (drill 0.8) (layers "*.Cu" "*.Mask") (remove_unused_layers no)
   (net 6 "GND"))
  (pad "262" thru_hole circle (at 31.75 -17.78) (size 2.54 2.54) (drill 0.8) (layers "*.Cu" "*.Mask") (remove_unused_layers no)
   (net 6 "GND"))
  (pad "263" thru_hole circle (at 34.29 -17.78) (size 2.54 2.54) (drill 0.8) (layers "*.Cu" "*.Mask") (remove_unused_layers no)
   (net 6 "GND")))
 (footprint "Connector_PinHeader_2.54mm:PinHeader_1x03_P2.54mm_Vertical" (layer "F.Cu") (at 49 91.92)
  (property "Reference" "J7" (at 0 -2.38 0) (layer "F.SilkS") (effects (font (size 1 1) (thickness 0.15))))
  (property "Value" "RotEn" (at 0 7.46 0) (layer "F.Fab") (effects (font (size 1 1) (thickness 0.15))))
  (pad "1" thru_hole rect (at 0 0) (size 1.7 1.7) (drill 1) (layers "*.Cu" "*.Mask") (remove_unused_layers no) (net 23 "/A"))
  (pad "2" thru_hole circle (at 0 2.54) (size 1.7 1.7) (drill 1) (layers "*.Cu" "*.Mask") (remove_unused_layers no) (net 25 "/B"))
  (pad "3" thru_hole circle (at 0 5.08) (size 1.7 1.7) (drill 1) (layers "*.Cu" "*.Mask") (remove_unused_layers no) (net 27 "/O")))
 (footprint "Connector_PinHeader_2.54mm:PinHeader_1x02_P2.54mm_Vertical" (layer "F.Cu") (at 154.5 82.04 180)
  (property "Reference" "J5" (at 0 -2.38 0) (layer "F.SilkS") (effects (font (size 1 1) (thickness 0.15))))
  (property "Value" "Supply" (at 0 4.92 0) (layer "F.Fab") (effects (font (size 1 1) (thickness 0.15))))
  (pad "1" thru_hole rect (at 0 0 180) (size 1.7 1.7) (drill 1) (layers "*.Cu" "*.Mask") (remove_unused_layers no) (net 7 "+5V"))
  (pad "2" thru_hole circle (at 0 2.54 180) (size 1.7 1.7) (drill 1) (layers "*.Cu" "*.Mask") (remove_unused_layers no) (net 6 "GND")))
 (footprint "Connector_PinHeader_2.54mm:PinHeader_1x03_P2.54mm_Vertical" (layer "F.Cu") (at 137.04 113.5 -90)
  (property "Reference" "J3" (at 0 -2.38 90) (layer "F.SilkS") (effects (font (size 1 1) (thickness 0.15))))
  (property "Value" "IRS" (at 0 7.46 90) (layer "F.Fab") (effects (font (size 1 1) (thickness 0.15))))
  (pad "1" thru_hole rect (at 0 0 270) (size 1.7 1.7) (drill 1) (layers "*.Cu" "*.Mask") (remove_unused_layers no) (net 7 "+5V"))
  (pad "2" thru_hole circle (at 0 2.54 270) (size 1.7 1.7) (drill 1) (layers "*.Cu" "*.Mask") (remove_unused_layers no) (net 6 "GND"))
  (pad "3" thru_hole circle (at 0 5.08 270) (size 1.7 1.7) (drill 1) (layers "*.Cu" "*.Mask") (remove_unused_layers no) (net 54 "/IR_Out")))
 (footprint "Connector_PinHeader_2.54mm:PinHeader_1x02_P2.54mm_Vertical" (layer "F.Cu") (at 155.5 100.225)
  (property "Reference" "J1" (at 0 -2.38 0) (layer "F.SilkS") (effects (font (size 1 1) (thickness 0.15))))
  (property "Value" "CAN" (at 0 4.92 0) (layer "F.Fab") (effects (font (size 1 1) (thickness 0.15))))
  (pad "1" thru_hole rect (at 0 0) (size 1.7 1.7) (drill 1) (layers "*.Cu" "*.Mask") (remove_unused_layers no) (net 10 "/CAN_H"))
  (pad "2" thru_hole circle (at 0 2.54) (size 1.7 1.7) (drill 1) (layers "*.Cu" "*.Mask") (remove_unused_layers no) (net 11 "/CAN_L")))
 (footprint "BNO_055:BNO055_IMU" (layer "F.Cu") (at 148.478 62.35 -90)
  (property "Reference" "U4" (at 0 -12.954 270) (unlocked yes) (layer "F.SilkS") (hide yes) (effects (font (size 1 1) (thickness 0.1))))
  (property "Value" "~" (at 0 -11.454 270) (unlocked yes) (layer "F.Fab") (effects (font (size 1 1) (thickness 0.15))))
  (pad "1" thru_hole circle (at -6.35 14.478 270) (size 2.54 2.54) (drill 0.8) (layers "*.Cu" "*.Mask") (remove_unused_layers no)
   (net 7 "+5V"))
  (pad "2" thru_hole circle (at -3.81 14.478 270) (size 2.54 2.54) (drill 0.8) (layers "*.Cu" "*.Mask") (remove_unused_layers no)
   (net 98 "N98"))
  (pad "3" thru_hole circle (at -1.27 14.478 270) (size 2.54 2.54) (drill 0.8) (layers "*.Cu" "*.Mask") (remove_unused_layers no)
   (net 6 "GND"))
  (pad "4" thru_hole circle (at 1.27 14.478 270) (size 2.54 2.54) (drill 0.8) (layers "*.Cu" "*.Mask") (remove_unused_layers no)
   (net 80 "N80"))
  (pad "5" thru_hole circle (at 3.81 14.478 270) (size 2.54 2.54) (drill 0.8) (layers "*.Cu" "*.Mask") (remove_unused_layers no)
   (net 81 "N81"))
  (pad "6" thru_hole circle (at 6.35 14.478 270) (size 2.54 2.54) (drill 0.8) (layers "*.Cu" "*.Mask") (remove_unused_layers no)
   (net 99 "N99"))
  (pad "7" thru_hole circle (at -3.81 -0.762 270) (size 2.54 2.54) (drill 0.8) (layers "*.Cu" "*.Mask") (remove_unused_layers no)
   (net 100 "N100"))
  (pad "8" thru_hole circle (at -1.27 -0.762 270) (size 2.54 2.54) (drill 0.8) (layers "*.Cu" "*.Mask") (remove_unused_layers no)
   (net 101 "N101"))
  (pad "9" thru_hole circle (at 1.27 -0.762 270) (size 2.54 2.54) (drill 0.8) (layers "*.Cu" "*.Mask") (remove_unused_layers no)
   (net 6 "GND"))
  (pad "10" thru_hole circle (at 3.81 -0.762 270) (size 2.54 2.54) (drill 0.8) (layers "*.Cu" "*.Mask") (remove_unused_layers no)
   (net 6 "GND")))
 (gr_rect (start 39 45.5) (end 157.5 135.5) (stroke (width 0.05) (type default)) (fill no) (layer "Edge.Cuts"))
 (segment (start 134 61.08) (end 152.42 79.5) (width 0.2) (layer "F.Cu") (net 6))
 (segment (start 52.475 78.18) (end 52.475 77.65) (width 0.2) (layer "F.Cu") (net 6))
 (segment (start 147.08127 79.5) (end 154.5 79.5) (width 0.2) (layer "F.Cu") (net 6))
 (segment (start 134.3171 128.052) (end 112.083 128.052) (width 0.2) (layer "F.Cu") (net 6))
 (segment (start 52.475 77.65) (end 58.33 71.795) (width 0.2) (layer "F.Cu") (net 6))
 (segment (start 131.467 104.956) (end 129.896 103.385) (width 0.2) (layer "F.Cu") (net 6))
 (segment (start 129.896 96.68527) (end 147.08127 79.5) (width 0.2) (layer "F.Cu") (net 6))
 (segment (start 112.083 128.052) (end 111.706 127.675) (width 0.2) (layer "F.Cu") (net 6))
 (segment (start 135.35 114.35) (end 135.35 127.0191) (width 0.2) (layer "F.Cu") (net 6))
 (segment (start 135.35 127.0191) (end 134.3171 128.052) (width 0.2) (layer "F.Cu") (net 6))
 (segment (start 134.5 113.5) (end 135.35 114.35) (width 0.2) (layer "F.Cu") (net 6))
 (segment (start 152.42 79.5) (end 154.5 79.5) (width 0.2) (layer "F.Cu") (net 6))
 (segment (start 129.896 103.385) (end 129.896 96.68527) (width 0.2) (layer "F.Cu") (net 6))
 (segment (start 151.787 102.416) (end 155.151 102.416) (width 0.2) (layer "F.Cu") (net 11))
 (segment (start 155.151 102.416) (end 155.5 102.765) (width 0.2) (layer "F.Cu") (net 11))
 (segment (start 155.151 99.876) (end 155.5 100.225) (width 0.2) (layer "F.Cu") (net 10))
 (segment (start 151.787 99.876) (end 155.151 99.876) (width 0.2) (layer "F.Cu") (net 10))
 (segment (start 133 126.145) (end 126.91 120.055) (width 0.2) (layer "F.Cu") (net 2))
 (segment (start 133 126.5) (end 133 126.145) (width 0.2) (layer "F.Cu") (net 2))
 (segment (start 131.96 113.5) (end 128.355 109.895) (width 0.2) (layer "F.Cu") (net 54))
 (segment (start 128.355 109.895) (end 126.91 109.895) (width 0.2) (layer "F.Cu") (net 54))
 (segment (start 137.04 113.5) (end 137.04 99.5) (width 0.2) (layer "F.Cu") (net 7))
 (segment (start 134 56) (end 154 56) (width 0.2) (layer "F.Cu") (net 7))
 (segment (start 152.44 84.1) (end 154.5 82.04) (width 0.2) (layer "F.Cu") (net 7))
 (segment (start 154 56) (end 156.5 58.5) (width 0.2) (layer "F.Cu") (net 7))
 (segment (start 139.204 97.336) (end 154.5 82.04) (width 0.2) (layer "F.Cu") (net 7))
 (segment (start 137.04 99.5) (end 154.5 82.04) (width 0.2) (layer "F.Cu") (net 7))
 (segment (start 131.467 97.336) (end 139.204 97.336) (width 0.2) (layer "F.Cu") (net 7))
 (segment (start 155.04 81.5) (end 154.5 82.04) (width 0.2) (layer "F.Cu") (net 7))
 (segment (start 156.5 58.5) (end 156.5 81.5) (width 0.2) (layer "F.Cu") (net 7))
 (segment (start 156.5 81.5) (end 155.04 81.5) (width 0.2) (layer "F.Cu") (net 7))
 (segment (start 50.923 66.82027) (end 57.67927 60.064) (width 0.2) (layer "F.Cu") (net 5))
 (segment (start 52.475 80.72) (end 50.923 79.168) (width 0.2) (layer "F.Cu") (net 5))
 (segment (start 50.923 79.168) (end 50.923 66.82027) (width 0.2) (layer "F.Cu") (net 5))
 (segment (start 57.67927 60.064) (end 62.064 60.064) (width 0.2) (layer "F.Cu") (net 5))
 (segment (start 62.064 60.064) (end 62.5 60.5) (width 0.2) (layer "F.Cu") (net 5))
 (segment (start 62.5 87.945) (end 60.87 89.575) (width 0.2) (layer "F.Cu") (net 5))
 (segment (start 62.5 60.5) (end 62.5 87.945) (width 0.2) (layer "F.Cu") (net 5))
 (segment (start 122.799 101.306) (end 124.37 99.735) (width 0.2) (layer "F.Cu") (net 8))
 (segment (start 134 120.198) (end 134.151 120.349) (width 0.2) (layer "F.Cu") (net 8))
 (segment (start 129.74427 127.651) (end 122.799 120.70573) (width 0.2) (layer "F.Cu") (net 8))
 (segment (start 131.467 99.876) (end 133.376 99.876) (width 0.2) (layer "F.Cu") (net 8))
 (segment (start 134.5 111.5) (end 133.349 112.651) (width 0.2) (layer "F.Cu") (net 8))
 (segment (start 134.151 120.349) (end 134.151 127.651) (width 0.2) (layer "F.Cu") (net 8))
 (segment (start 133.349 114.849) (end 134 115.5) (width 0.2) (layer "F.Cu") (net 8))
 (segment (start 134.151 127.651) (end 129.74427 127.651) (width 0.2) (layer "F.Cu") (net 8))
 (segment (start 134 115.5) (end 134 120.198) (width 0.2) (layer "F.Cu") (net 8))
 (segment (start 134.5 101) (end 134.5 111.5) (width 0.2) (layer "F.Cu") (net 8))
 (segment (start 122.799 120.70573) (end 122.799 101.306) (width 0.2) (layer "F.Cu") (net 8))
 (segment (start 133.349 112.651) (end 133.349 114.849) (width 0.2) (layer "F.Cu") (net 8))
 (segment (start 133.376 99.876) (end 134.5 101) (width 0.2) (layer "F.Cu") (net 8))
 (segment (start 128.5 101.325) (end 126.91 99.735) (width 0.2) (layer "F.Cu") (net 9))
 (segment (start 132.973 106.527) (end 128.527 106.527) (width 0.2) (layer "F.Cu") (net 9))
 (segment (start 133.038 103.987) (end 133.038 106.462) (width 0.2) (layer "F.Cu") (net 9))
 (segment (start 128.5 106.5) (end 128.5 101.325) (width 0.2) (layer "F.Cu") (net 9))
 (segment (start 131.467 102.416) (end 133.038 103.987) (width 0.2) (layer "F.Cu") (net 9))
 (segment (start 128.527 106.527) (end 128.5 106.5) (width 0.2) (layer "F.Cu") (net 9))
 (segment (start 133.038 106.462) (end 132.973 106.527) (width 0.2) (layer "F.Cu") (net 9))
 (segment (start 51.324 84.411) (end 51.324 86.951) (width 0.2) (layer "F.Cu") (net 4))
 (segment (start 53.948 89.575) (end 58.33 89.575) (width 0.2) (layer "F.Cu") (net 4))
 (segment (start 51.324 86.951) (end 53.948 89.575) (width 0.2) (layer "F.Cu") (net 4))
 (segment (start 52.475 83.26) (end 51.324 84.411) (width 0.2) (layer "F.Cu") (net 4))
 (segment (start 133 121.5) (end 130.895 121.5) (width 0.2) (layer "F.Cu") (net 1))
 (segment (start 130.895 121.5) (end 126.91 117.515) (width 0.2) (layer "F.Cu") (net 1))
 (segment (start 51.324 71.181) (end 58.33 64.175) (width 0.2) (layer "F.Cu") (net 3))
 (segment (start 51.324 78.65676) (end 51.324 71.181) (width 0.2) (layer "F.Cu") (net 3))
 (segment (start 52.475 85.8) (end 53.626 84.649) (width 0.2) (layer "F.Cu") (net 3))
 (segment (start 53.626 84.649) (end 53.626 80.126) (width 0.2) (layer "F.Cu") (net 3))
 (segment (start 52.16724 79.5) (end 51.324 78.65676) (width 0.2) (layer "F.Cu") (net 3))
 (segment (start 53 79.5) (end 52.16724 79.5) (width 0.2) (layer "F.Cu") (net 3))
 (segment (start 53.626 80.126) (end 53 79.5) (width 0.2) (layer "F.Cu") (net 3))
 (segment (start 123.71927 60.064) (end 122.799 60.98427) (width 0.2) (layer "F.Cu") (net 81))
 (segment (start 134 66.16) (end 127.904 60.064) (width 0.2) (layer "F.Cu") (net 81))
 (segment (start 127.904 60.064) (end 123.71927 60.064) (width 0.2) (layer "F.Cu") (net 81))
 (segment (start 122.799 75.304) (end 124.37 76.875) (width 0.2) (layer "F.Cu") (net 81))
 (segment (start 122.799 60.98427) (end 122.799 75.304) (width 0.2) (layer "F.Cu") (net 81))
 (segment (start 131.125 76.875) (end 126.91 76.875) (width 0.2) (layer "F.Cu") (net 80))
 (segment (start 135.571 72.429) (end 131.125 76.875) (width 0.2) (layer "F.Cu") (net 80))
 (segment (start 135.571 65.191) (end 135.571 72.429) (width 0.2) (layer "F.Cu") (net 80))
 (segment (start 134 63.62) (end 135.571 65.191) (width 0.2) (layer "F.Cu") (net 80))
 (segment (start 58.135 94.46) (end 58.33 94.655) (width 0.2) (layer "F.Cu") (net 25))
 (segment (start 49 94.46) (end 58.135 94.46) (width 0.2) (layer "F.Cu") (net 25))
 (segment (start 49 97) (end 58.135 97) (width 0.2) (layer "F.Cu") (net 27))
 (segment (start 58.135 97) (end 58.33 97.195) (width 0.2) (layer "F.Cu") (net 27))
 (segment (start 49 91.92) (end 58.135 91.92) (width 0.2) (layer "F.Cu") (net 23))
 (segment (start 58.135 91.92) (end 58.33 92.115) (width 0.2) (layer "F.Cu") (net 23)))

